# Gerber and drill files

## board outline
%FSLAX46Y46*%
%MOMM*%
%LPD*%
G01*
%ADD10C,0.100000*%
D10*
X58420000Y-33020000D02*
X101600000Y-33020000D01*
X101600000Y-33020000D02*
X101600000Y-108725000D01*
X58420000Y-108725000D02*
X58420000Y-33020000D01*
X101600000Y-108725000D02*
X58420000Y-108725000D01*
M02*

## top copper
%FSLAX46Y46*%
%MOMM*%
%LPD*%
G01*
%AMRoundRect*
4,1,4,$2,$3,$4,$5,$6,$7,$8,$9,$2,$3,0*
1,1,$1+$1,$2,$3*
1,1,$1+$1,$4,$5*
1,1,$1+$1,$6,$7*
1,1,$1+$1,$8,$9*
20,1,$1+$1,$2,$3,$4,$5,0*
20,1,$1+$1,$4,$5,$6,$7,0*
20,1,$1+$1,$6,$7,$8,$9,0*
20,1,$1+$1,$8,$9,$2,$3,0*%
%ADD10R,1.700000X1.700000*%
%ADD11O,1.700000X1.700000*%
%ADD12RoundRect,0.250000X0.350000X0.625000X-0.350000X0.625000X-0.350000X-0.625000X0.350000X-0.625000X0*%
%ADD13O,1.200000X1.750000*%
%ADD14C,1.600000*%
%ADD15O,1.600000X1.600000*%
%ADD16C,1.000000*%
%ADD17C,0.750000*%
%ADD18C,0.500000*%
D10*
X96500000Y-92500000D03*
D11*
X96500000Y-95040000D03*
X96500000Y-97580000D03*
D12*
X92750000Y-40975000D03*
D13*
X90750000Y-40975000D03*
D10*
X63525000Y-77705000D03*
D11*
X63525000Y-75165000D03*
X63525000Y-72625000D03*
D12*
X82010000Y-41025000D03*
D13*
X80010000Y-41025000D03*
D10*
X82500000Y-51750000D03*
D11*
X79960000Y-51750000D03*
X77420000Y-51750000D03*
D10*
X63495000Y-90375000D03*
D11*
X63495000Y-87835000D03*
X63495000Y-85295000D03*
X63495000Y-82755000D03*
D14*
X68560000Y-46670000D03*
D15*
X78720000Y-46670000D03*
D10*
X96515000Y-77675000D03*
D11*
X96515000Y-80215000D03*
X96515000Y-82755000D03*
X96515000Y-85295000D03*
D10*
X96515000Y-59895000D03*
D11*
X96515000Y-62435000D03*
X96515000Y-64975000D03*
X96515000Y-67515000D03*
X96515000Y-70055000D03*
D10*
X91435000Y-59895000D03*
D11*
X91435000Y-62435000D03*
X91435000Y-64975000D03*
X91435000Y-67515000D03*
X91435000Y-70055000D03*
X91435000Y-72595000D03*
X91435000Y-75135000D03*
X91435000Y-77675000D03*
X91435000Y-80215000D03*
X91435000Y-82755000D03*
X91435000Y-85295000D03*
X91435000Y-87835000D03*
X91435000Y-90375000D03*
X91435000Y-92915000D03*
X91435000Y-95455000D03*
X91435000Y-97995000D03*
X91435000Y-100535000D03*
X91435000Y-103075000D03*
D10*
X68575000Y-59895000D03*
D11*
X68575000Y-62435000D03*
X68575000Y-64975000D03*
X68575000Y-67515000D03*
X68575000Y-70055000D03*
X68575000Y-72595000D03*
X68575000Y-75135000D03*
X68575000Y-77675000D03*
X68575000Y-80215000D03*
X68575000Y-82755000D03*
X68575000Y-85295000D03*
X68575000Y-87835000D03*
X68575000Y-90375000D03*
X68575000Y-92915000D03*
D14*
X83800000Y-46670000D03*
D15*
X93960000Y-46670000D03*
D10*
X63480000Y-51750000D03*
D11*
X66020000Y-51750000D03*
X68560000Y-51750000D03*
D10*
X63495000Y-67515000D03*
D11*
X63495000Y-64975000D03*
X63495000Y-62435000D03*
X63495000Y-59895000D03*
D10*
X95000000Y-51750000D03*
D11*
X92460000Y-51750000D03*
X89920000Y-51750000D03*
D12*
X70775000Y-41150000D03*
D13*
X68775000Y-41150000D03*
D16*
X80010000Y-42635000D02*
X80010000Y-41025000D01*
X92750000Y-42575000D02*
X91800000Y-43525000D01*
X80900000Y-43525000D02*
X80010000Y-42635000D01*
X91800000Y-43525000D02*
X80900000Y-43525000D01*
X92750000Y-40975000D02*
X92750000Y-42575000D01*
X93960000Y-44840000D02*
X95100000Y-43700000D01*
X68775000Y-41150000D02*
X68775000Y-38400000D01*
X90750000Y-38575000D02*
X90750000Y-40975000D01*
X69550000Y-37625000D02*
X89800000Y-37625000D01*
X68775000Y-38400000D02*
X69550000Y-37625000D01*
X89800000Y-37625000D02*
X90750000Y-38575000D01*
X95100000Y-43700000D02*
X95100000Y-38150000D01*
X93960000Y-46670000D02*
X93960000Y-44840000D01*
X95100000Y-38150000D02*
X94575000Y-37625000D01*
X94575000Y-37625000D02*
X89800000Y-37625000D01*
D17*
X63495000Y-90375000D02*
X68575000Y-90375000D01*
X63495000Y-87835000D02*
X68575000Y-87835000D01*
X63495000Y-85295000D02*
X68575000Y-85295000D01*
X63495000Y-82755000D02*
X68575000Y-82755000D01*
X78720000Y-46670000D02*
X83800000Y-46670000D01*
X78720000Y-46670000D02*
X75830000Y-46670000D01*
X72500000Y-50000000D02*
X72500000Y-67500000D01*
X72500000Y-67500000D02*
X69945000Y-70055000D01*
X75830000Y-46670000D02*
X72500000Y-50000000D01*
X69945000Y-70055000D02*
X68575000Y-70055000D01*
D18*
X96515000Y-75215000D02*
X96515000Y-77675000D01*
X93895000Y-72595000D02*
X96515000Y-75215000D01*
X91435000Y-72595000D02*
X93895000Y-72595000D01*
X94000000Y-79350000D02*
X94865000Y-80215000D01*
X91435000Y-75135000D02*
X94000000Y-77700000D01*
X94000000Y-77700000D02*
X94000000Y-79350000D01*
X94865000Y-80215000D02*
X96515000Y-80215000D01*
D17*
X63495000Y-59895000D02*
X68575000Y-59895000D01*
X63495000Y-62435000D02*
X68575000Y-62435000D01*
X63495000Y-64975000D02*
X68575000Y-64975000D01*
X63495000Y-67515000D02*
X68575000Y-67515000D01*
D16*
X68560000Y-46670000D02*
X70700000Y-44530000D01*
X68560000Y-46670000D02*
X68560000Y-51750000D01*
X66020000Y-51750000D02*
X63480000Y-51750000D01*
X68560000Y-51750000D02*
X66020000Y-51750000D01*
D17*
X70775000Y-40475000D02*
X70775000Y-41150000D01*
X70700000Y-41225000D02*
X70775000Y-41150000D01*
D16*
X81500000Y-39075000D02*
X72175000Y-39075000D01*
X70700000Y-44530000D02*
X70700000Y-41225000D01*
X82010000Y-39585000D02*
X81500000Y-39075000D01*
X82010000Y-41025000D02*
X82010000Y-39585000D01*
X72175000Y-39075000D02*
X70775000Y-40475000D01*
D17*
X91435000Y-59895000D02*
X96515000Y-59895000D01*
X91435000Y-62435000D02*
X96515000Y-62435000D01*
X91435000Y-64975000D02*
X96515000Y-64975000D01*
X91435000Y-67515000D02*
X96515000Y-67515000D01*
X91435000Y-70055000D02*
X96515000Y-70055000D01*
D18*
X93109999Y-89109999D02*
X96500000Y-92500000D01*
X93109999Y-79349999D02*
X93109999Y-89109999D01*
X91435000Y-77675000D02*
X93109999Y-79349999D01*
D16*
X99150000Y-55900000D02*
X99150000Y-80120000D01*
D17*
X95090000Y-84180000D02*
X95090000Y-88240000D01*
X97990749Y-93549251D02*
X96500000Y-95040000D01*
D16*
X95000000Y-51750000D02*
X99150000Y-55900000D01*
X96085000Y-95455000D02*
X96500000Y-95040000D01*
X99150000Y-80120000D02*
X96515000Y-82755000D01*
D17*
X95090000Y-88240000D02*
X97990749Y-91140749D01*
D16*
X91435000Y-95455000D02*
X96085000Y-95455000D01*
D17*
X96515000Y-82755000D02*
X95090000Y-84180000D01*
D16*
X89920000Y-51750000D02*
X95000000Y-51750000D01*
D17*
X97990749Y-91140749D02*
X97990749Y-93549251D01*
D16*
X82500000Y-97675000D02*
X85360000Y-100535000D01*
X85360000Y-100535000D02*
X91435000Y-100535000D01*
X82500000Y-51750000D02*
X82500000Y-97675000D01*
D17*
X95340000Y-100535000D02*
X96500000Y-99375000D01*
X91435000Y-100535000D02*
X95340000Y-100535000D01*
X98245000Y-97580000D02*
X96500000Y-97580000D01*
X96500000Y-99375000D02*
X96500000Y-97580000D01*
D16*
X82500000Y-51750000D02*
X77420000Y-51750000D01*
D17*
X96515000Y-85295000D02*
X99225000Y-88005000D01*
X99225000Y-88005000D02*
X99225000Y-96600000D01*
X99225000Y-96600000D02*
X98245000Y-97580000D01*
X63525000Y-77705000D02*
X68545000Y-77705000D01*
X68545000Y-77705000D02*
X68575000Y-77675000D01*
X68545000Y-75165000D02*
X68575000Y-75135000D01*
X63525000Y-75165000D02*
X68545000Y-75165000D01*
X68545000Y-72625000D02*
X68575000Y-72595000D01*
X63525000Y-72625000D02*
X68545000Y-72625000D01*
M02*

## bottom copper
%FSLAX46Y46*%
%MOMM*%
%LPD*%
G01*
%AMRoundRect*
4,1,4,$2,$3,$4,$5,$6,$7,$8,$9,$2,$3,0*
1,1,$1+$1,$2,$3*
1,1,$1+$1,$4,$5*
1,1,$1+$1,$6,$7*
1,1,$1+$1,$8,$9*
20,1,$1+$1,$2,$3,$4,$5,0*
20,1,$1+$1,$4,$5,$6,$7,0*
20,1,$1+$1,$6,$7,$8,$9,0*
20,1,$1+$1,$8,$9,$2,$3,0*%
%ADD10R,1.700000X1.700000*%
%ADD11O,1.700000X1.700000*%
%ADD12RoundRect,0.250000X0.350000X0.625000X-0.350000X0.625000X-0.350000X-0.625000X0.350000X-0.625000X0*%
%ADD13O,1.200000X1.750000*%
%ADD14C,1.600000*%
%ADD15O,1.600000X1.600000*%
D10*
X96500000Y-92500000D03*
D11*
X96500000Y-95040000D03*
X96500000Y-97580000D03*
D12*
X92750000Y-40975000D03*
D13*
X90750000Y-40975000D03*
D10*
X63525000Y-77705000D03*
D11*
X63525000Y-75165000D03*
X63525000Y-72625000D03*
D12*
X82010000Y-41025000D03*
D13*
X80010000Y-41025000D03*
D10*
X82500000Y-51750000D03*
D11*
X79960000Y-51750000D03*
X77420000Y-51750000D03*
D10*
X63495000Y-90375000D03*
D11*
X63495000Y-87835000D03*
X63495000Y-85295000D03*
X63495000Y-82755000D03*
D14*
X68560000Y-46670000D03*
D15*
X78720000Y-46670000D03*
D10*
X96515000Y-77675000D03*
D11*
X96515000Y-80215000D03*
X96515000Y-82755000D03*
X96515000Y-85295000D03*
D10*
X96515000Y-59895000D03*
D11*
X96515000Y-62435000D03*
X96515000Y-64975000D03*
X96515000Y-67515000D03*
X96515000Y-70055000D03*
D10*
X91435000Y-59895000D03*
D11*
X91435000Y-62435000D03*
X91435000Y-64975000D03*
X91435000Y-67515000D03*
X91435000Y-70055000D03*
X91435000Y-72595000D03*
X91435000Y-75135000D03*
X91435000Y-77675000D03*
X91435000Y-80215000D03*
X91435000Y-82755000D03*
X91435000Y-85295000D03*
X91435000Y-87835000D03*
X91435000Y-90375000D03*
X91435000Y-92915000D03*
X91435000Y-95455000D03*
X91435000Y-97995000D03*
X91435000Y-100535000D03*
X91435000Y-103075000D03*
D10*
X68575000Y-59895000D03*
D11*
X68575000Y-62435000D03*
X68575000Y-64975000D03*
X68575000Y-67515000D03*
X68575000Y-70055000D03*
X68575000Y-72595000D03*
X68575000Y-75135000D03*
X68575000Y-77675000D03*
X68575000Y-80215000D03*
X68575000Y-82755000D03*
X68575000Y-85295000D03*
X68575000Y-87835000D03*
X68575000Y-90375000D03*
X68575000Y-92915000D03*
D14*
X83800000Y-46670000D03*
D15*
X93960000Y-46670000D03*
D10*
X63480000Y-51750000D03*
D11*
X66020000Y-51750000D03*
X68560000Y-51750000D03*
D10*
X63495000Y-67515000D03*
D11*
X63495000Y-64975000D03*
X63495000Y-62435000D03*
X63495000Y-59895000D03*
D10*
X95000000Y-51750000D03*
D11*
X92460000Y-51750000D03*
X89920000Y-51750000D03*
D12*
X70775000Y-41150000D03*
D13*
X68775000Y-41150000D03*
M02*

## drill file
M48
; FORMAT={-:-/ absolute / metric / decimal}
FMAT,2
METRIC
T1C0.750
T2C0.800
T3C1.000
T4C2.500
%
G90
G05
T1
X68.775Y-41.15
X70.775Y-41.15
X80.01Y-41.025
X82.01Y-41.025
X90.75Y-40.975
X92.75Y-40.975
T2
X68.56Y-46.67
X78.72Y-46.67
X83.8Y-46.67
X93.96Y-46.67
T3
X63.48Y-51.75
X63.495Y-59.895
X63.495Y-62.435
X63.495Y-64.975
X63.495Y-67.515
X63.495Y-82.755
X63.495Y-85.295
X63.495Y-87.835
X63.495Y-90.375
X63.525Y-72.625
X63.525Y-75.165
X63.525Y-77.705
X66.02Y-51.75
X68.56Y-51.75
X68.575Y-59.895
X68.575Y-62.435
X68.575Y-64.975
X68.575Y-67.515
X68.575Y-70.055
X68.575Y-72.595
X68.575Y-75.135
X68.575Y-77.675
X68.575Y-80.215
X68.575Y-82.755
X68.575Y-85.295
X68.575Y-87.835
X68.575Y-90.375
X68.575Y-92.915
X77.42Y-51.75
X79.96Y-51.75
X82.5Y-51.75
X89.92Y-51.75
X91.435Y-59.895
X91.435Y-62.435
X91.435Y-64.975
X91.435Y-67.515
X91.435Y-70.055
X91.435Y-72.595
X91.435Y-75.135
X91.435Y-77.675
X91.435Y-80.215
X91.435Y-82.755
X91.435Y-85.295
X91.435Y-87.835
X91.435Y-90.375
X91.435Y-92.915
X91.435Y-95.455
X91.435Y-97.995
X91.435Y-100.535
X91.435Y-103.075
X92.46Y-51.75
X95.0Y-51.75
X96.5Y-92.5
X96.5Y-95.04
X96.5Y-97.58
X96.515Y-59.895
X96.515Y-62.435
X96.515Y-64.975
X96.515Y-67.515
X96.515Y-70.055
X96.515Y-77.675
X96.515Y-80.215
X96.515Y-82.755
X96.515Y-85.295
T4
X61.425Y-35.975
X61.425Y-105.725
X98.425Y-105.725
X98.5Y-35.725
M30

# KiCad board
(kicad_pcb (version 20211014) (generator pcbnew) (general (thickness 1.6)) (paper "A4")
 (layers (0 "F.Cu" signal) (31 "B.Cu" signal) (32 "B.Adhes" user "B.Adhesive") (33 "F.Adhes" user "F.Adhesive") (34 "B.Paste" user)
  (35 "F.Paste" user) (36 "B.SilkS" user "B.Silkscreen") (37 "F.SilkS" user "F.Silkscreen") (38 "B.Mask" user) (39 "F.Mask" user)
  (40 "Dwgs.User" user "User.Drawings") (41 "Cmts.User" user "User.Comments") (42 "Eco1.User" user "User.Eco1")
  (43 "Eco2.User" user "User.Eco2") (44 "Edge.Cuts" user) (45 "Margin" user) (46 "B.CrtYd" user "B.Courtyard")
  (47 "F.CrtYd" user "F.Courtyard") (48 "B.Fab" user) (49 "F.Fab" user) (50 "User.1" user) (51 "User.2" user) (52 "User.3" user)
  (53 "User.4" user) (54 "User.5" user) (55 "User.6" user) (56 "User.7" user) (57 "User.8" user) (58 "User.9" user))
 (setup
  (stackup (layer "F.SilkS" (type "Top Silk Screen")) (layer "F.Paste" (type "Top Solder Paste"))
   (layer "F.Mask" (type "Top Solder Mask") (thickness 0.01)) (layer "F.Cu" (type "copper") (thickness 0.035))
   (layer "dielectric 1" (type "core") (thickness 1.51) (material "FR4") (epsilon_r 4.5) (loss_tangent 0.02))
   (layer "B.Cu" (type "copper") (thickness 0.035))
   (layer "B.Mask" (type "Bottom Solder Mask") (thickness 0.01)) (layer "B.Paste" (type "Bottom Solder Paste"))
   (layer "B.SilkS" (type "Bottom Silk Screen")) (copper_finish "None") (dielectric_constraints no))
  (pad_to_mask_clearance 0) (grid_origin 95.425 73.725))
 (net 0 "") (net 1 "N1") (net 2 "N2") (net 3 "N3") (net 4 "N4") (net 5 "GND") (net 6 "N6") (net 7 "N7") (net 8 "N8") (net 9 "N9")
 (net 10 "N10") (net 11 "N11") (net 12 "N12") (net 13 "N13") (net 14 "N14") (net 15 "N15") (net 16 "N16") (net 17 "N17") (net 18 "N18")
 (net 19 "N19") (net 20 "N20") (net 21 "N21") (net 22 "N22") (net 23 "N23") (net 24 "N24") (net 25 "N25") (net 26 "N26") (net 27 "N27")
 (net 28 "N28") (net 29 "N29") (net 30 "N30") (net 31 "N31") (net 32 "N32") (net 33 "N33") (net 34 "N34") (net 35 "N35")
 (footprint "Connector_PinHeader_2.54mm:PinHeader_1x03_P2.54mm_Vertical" (layer "F.Cu") (at 96.5 92.5)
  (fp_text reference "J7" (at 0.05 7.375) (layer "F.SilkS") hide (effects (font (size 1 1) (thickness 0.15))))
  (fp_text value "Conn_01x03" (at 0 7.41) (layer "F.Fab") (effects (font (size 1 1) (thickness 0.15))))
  (pad "1" thru_hole rect (at 0 0) (size 1.7 1.7) (drill 1) (layers *.Cu *.Mask) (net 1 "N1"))
  (pad "2" thru_hole oval (at 0 2.54) (size 1.7 1.7) (drill 1) (layers *.Cu *.Mask) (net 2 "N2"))
  (pad "3" thru_hole oval (at 0 5.08) (size 1.7 1.7) (drill 1) (layers *.Cu *.Mask) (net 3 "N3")))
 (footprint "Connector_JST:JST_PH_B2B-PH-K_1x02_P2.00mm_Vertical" (layer "F.Cu") (at 92.75 40.975 180)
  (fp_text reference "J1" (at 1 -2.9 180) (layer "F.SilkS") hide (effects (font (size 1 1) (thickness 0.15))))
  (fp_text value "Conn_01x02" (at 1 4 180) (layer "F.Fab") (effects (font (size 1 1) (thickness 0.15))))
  (pad "1" thru_hole roundrect (at 0 0 180) (size 1.2 1.75) (drill 0.75) (layers *.Cu *.Mask) (roundrect_rratio 0.208333) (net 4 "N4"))
  (pad "2" thru_hole oval (at 2 0 180) (size 1.2 1.75) (drill 0.75) (layers *.Cu *.Mask) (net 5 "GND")))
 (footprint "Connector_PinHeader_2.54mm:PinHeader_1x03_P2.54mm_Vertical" (layer "F.Cu") (at 63.525 77.705 180)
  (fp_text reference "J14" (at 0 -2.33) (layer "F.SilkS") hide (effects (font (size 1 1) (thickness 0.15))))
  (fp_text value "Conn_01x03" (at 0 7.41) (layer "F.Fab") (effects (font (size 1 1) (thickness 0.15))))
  (pad "1" thru_hole rect (at 0 0 180) (size 1.7 1.7) (drill 1) (layers *.Cu *.Mask) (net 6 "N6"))
  (pad "2" thru_hole oval (at 0 2.54 180) (size 1.7 1.7) (drill 1) (layers *.Cu *.Mask) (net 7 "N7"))
  (pad "3" thru_hole oval (at 0 5.08 180) (size 1.7 1.7) (drill 1) (layers *.Cu *.Mask) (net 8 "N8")))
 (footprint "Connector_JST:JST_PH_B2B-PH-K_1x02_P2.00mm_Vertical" (layer "F.Cu") (at 82.01 41.025 180)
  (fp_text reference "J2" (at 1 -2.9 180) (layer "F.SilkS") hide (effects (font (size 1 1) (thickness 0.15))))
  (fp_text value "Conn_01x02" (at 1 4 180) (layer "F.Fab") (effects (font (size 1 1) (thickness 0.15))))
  (pad "1" thru_hole roundrect (at 0 0 180) (size 1.2 1.75) (drill 0.75) (layers *.Cu *.Mask) (roundrect_rratio 0.208333) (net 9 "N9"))
  (pad "2" thru_hole oval (at 2 0 180) (size 1.2 1.75) (drill 0.75) (layers *.Cu *.Mask) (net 4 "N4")))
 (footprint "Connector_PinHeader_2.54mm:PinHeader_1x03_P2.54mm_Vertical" (layer "F.Cu") (at 82.5 51.75 -90)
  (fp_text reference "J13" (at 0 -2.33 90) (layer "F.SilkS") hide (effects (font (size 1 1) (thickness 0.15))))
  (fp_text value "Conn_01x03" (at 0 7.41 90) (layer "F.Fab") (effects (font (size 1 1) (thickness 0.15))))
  (pad "1" thru_hole rect (at 0 0 270) (size 1.7 1.7) (drill 1) (layers *.Cu *.Mask) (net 3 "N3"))
  (pad "2" thru_hole oval (at 0 2.54 270) (size 1.7 1.7) (drill 1) (layers *.Cu *.Mask) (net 3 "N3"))
  (pad "3" thru_hole oval (at 0 5.08 270) (size 1.7 1.7) (drill 1) (layers *.Cu *.Mask) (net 3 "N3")))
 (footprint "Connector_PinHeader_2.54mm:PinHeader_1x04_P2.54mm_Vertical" (layer "F.Cu") (at 63.495 90.375 180)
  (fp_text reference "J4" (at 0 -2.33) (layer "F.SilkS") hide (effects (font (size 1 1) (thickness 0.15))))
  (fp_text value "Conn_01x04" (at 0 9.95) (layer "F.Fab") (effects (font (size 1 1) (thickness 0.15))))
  (pad "1" thru_hole rect (at 0 0 180) (size 1.7 1.7) (drill 1) (layers *.Cu *.Mask) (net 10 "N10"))
  (pad "2" thru_hole oval (at 0 2.54 180) (size 1.7 1.7) (drill 1) (layers *.Cu *.Mask) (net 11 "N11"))
  (pad "3" thru_hole oval (at 0 5.08 180) (size 1.7 1.7) (drill 1) (layers *.Cu *.Mask) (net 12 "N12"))
  (pad "4" thru_hole oval (at 0 7.62 180) (size 1.7 1.7) (drill 1) (layers *.Cu *.Mask) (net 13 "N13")))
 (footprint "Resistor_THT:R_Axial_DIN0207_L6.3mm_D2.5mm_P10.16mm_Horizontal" (layer "F.Cu") (at 68.56 46.67)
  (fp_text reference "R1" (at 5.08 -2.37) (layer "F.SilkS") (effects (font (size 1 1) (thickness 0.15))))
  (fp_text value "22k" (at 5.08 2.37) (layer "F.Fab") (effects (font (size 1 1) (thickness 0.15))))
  (pad "1" thru_hole circle (at 0 0) (size 1.6 1.6) (drill 0.8) (layers *.Cu *.Mask) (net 9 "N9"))
  (pad "2" thru_hole oval (at 10.16 0) (size 1.6 1.6) (drill 0.8) (layers *.Cu *.Mask) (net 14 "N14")))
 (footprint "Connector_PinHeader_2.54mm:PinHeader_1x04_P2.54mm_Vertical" (layer "F.Cu") (at 96.515 77.675)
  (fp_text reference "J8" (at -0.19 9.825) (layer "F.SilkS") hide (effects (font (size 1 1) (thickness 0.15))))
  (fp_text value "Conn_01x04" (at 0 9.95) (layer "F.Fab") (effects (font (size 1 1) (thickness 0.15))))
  (pad "1" thru_hole rect (at 0 0) (size 1.7 1.7) (drill 1) (layers *.Cu *.Mask) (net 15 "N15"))
  (pad "2" thru_hole oval (at 0 2.54) (size 1.7 1.7) (drill 1) (layers *.Cu *.Mask) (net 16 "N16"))
  (pad "3" thru_hole oval (at 0 5.08) (size 1.7 1.7) (drill 1) (layers *.Cu *.Mask) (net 2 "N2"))
  (pad "4" thru_hole oval (at 0 7.62) (size 1.7 1.7) (drill 1) (layers *.Cu *.Mask) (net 3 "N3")))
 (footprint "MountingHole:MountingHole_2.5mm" (layer "F.Cu") (at 98.425 35.725)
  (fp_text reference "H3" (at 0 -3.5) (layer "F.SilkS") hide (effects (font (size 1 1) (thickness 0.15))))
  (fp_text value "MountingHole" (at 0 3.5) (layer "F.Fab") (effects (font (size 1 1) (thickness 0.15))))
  (pad "" np_thru_hole circle (at 0.075 0) (size 2.5 2.5) (drill 2.5) (layers F&B.Cu *.Mask)))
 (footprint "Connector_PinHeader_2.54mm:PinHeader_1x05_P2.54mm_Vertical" (layer "F.Cu") (at 96.515 59.895)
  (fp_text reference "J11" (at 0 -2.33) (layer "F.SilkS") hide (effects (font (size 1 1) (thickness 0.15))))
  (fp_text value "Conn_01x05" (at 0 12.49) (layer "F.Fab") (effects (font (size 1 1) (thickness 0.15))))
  (pad "1" thru_hole rect (at 0 0) (size 1.7 1.7) (drill 1) (layers *.Cu *.Mask) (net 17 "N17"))
  (pad "2" thru_hole oval (at 0 2.54) (size 1.7 1.7) (drill 1) (layers *.Cu *.Mask) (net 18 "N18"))
  (pad "3" thru_hole oval (at 0 5.08) (size 1.7 1.7) (drill 1) (layers *.Cu *.Mask) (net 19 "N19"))
  (pad "4" thru_hole oval (at 0 7.62) (size 1.7 1.7) (drill 1) (layers *.Cu *.Mask) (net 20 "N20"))
  (pad "5" thru_hole oval (at 0 10.16) (size 1.7 1.7) (drill 1) (layers *.Cu *.Mask) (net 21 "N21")))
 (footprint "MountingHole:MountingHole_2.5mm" (layer "F.Cu") (at 61.425 35.975)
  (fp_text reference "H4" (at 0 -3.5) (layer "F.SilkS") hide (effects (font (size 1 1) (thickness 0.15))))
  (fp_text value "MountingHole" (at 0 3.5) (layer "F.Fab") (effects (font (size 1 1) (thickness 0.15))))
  (pad "" np_thru_hole circle (at 0 0) (size 2.5 2.5) (drill 2.5) (layers *.Cu *.Mask)))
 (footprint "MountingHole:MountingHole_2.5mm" (layer "F.Cu") (at 98.425 105.725)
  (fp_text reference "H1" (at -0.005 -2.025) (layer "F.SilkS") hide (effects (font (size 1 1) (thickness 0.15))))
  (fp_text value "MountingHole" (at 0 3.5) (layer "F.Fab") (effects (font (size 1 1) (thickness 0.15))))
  (pad "" np_thru_hole circle (at 0 0) (size 2.5 2.5) (drill 2.5) (layers *.Cu *.Mask)))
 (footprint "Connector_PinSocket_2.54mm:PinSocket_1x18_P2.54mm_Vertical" (layer "F.Cu") (at 91.435 59.895)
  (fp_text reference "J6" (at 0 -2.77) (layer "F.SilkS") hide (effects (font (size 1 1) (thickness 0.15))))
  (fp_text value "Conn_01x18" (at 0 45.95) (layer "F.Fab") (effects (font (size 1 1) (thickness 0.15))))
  (pad "1" thru_hole rect (at 0 0) (size 1.7 1.7) (drill 1) (layers *.Cu *.Mask) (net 17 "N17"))
  (pad "2" thru_hole oval (at 0 2.54) (size 1.7 1.7) (drill 1) (layers *.Cu *.Mask) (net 18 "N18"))
  (pad "3" thru_hole oval (at 0 5.08) (size 1.7 1.7) (drill 1) (layers *.Cu *.Mask) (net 19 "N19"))
  (pad "4" thru_hole oval (at 0 7.62) (size 1.7 1.7) (drill 1) (layers *.Cu *.Mask) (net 20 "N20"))
  (pad "5" thru_hole oval (at 0 10.16) (size 1.7 1.7) (drill 1) (layers *.Cu *.Mask) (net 21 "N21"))
  (pad "6" thru_hole oval (at 0 12.7) (size 1.7 1.7) (drill 1) (layers *.Cu *.Mask) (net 15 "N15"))
  (pad "7" thru_hole oval (at 0 15.24) (size 1.7 1.7) (drill 1) (layers *.Cu *.Mask) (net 16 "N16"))
  (pad "8" thru_hole oval (at 0 17.78) (size 1.7 1.7) (drill 1) (layers *.Cu *.Mask) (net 1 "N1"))
  (pad "9" thru_hole oval (at 0 20.32) (size 1.7 1.7) (drill 1) (layers *.Cu *.Mask) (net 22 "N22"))
  (pad "10" thru_hole oval (at 0 22.86) (size 1.7 1.7) (drill 1) (layers *.Cu *.Mask) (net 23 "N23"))
  (pad "11" thru_hole oval (at 0 25.4) (size 1.7 1.7) (drill 1) (layers *.Cu *.Mask) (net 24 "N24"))
  (pad "12" thru_hole oval (at 0 27.94) (size 1.7 1.7) (drill 1) (layers *.Cu *.Mask) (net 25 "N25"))
  (pad "13" thru_hole oval (at 0 30.48) (size 1.7 1.7) (drill 1) (layers *.Cu *.Mask) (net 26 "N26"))
  (pad "14" thru_hole oval (at 0 33.02) (size 1.7 1.7) (drill 1) (layers *.Cu *.Mask) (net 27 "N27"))
  (pad "15" thru_hole oval (at 0 35.56) (size 1.7 1.7) (drill 1) (layers *.Cu *.Mask) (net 2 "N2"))
  (pad "16" thru_hole oval (at 0 38.1) (size 1.7 1.7) (drill 1) (layers *.Cu *.Mask) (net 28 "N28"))
  (pad "17" thru_hole oval (at 0 40.64) (size 1.7 1.7) (drill 1) (layers *.Cu *.Mask) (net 3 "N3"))
  (pad "18" thru_hole oval (at 0 43.18) (size 1.7 1.7) (drill 1) (layers *.Cu *.Mask) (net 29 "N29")))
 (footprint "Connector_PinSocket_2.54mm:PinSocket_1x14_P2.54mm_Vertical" (layer "F.Cu") (at 68.575 59.895)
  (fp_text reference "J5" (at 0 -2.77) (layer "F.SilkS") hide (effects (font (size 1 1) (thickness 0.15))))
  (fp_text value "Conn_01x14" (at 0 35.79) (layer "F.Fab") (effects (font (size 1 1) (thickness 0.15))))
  (pad "1" thru_hole rect (at 0 0) (size 1.7 1.7) (drill 1) (layers *.Cu *.Mask) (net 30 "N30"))
  (pad "2" thru_hole oval (at 0 2.54) (size 1.7 1.7) (drill 1) (layers *.Cu *.Mask) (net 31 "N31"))
  (pad "3" thru_hole oval (at 0 5.08) (size 1.7 1.7) (drill 1) (layers *.Cu *.Mask) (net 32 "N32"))
  (pad "4" thru_hole oval (at 0 7.62) (size 1.7 1.7) (drill 1) (layers *.Cu *.Mask) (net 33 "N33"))
  (pad "5" thru_hole oval (at 0 10.16) (size 1.7 1.7) (drill 1) (layers *.Cu *.Mask) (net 14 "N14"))
  (pad "6" thru_hole oval (at 0 12.7) (size 1.7 1.7) (drill 1) (layers *.Cu *.Mask) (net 8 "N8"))
  (pad "7" thru_hole oval (at 0 15.24) (size 1.7 1.7) (drill 1) (layers *.Cu *.Mask) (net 7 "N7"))
  (pad "8" thru_hole oval (at 0 17.78) (size 1.7 1.7) (drill 1) (layers *.Cu *.Mask) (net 6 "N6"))
  (pad "9" thru_hole oval (at 0 20.32) (size 1.7 1.7) (drill 1) (layers *.Cu *.Mask) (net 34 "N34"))
  (pad "10" thru_hole oval (at 0 22.86) (size 1.7 1.7) (drill 1) (layers *.Cu *.Mask) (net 13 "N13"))
  (pad "11" thru_hole oval (at 0 25.4) (size 1.7 1.7) (drill 1) (layers *.Cu *.Mask) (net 12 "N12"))
  (pad "12" thru_hole oval (at 0 27.94) (size 1.7 1.7) (drill 1) (layers *.Cu *.Mask) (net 11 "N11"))
  (pad "13" thru_hole oval (at 0 30.48) (size 1.7 1.7) (drill 1) (layers *.Cu *.Mask) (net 10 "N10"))
  (pad "14" thru_hole oval (at 0 33.02) (size 1.7 1.7) (drill 1) (layers *.Cu *.Mask) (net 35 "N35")))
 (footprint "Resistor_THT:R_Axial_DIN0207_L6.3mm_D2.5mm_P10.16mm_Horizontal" (layer "F.Cu") (at 83.8 46.67)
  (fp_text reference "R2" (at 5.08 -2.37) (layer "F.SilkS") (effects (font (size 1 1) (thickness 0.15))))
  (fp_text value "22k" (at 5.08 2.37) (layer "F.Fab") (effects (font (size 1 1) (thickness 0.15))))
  (pad "1" thru_hole circle (at 0 0) (size 1.6 1.6) (drill 0.8) (layers *.Cu *.Mask) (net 14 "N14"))
  (pad "2" thru_hole oval (at 10.16 0) (size 1.6 1.6) (drill 0.8) (layers *.Cu *.Mask) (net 5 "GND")))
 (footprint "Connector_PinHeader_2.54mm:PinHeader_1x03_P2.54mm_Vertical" (layer "F.Cu") (at 63.48 51.75 90)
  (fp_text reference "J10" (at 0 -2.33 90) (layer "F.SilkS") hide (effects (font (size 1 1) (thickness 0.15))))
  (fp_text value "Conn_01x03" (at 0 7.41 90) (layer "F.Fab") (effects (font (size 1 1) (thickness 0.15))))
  (pad "1" thru_hole rect (at 0 0 90) (size 1.7 1.7) (drill 1) (layers *.Cu *.Mask) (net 9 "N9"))
  (pad "2" thru_hole oval (at 0 2.54 90) (size 1.7 1.7) (drill 1) (layers *.Cu *.Mask) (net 9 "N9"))
  (pad "3" thru_hole oval (at 0 5.08 90) (size 1.7 1.7) (drill 1) (layers *.Cu *.Mask) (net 9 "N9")))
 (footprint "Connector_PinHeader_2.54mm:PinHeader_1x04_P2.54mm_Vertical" (layer "F.Cu") (at 63.495 67.515 180)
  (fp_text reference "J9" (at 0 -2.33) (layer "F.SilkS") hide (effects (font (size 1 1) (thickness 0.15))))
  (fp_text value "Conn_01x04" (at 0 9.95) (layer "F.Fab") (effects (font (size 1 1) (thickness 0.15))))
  (pad "1" thru_hole rect (at 0 0 180) (size 1.7 1.7) (drill 1) (layers *.Cu *.Mask) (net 33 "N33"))
  (pad "2" thru_hole oval (at 0 2.54 180) (size 1.7 1.7) (drill 1) (layers *.Cu *.Mask) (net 32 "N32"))
  (pad "3" thru_hole oval (at 0 5.08 180) (size 1.7 1.7) (drill 1) (layers *.Cu *.Mask) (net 31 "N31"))
  (pad "4" thru_hole oval (at 0 7.62 180) (size 1.7 1.7) (drill 1) (layers *.Cu *.Mask) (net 30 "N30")))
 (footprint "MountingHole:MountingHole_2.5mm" (layer "F.Cu") (at 61.425 105.725)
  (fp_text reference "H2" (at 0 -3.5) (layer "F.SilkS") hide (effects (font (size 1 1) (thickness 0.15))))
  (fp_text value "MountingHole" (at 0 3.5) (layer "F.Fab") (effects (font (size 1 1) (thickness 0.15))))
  (pad "" np_thru_hole circle (at 0 0) (size 2.5 2.5) (drill 2.5) (layers *.Cu *.Mask)))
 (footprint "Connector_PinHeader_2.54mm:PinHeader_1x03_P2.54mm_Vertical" (layer "F.Cu") (at 95 51.75 -90)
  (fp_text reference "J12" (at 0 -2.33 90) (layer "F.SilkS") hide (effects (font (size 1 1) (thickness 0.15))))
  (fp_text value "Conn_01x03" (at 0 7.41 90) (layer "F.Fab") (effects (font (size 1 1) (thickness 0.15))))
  (pad "1" thru_hole rect (at 0 0 270) (size 1.7 1.7) (drill 1) (layers *.Cu *.Mask) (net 2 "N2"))
  (pad "2" thru_hole oval (at 0 2.54 270) (size 1.7 1.7) (drill 1) (layers *.Cu *.Mask) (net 2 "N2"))
  (pad "3" thru_hole oval (at 0 5.08 270) (size 1.7 1.7) (drill 1) (layers *.Cu *.Mask) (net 2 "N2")))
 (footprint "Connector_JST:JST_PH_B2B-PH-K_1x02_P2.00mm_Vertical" (layer "F.Cu") (at 70.775 41.15 180)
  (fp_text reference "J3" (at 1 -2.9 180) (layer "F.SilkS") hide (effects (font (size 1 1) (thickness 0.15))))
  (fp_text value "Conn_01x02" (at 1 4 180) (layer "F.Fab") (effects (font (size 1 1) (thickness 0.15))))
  (pad "1" thru_hole roundrect (at 0 0 180) (size 1.2 1.75) (drill 0.75) (layers *.Cu *.Mask) (roundrect_rratio 0.208333) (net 9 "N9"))
  (pad "2" thru_hole oval (at 2 0 180) (size 1.2 1.75) (drill 0.75) (layers *.Cu *.Mask) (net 5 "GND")))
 (gr_line (start 58.42 33.02) (end 101.6 33.02) (layer "Edge.Cuts") (width 0.1))
 (gr_line (start 101.6 33.02) (end 101.6 108.725) (layer "Edge.Cuts") (width 0.1))
 (gr_line (start 58.42 108.725) (end 58.42 33.02) (layer "Edge.Cuts") (width 0.1))
 (gr_line (start 101.6 108.725) (end 58.42 108.725) (layer "Edge.Cuts") (width 0.1))
 (segment (start 80.01 42.635) (end 80.01 41.025) (width 1) (layer "F.Cu") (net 4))
 (segment (start 92.75 42.575) (end 91.8 43.525) (width 1) (layer "F.Cu") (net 4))
 (segment (start 80.9 43.525) (end 80.01 42.635) (width 1) (layer "F.Cu") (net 4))
 (segment (start 91.8 43.525) (end 80.9 43.525) (width 1) (layer "F.Cu") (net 4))
 (segment (start 92.75 40.975) (end 92.75 42.575) (width 1) (layer "F.Cu") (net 4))
 (segment (start 93.96 44.84) (end 95.1 43.7) (width 1) (layer "F.Cu") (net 5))
 (segment (start 68.775 41.15) (end 68.775 38.4) (width 1) (layer "F.Cu") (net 5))
 (segment (start 90.75 38.575) (end 90.75 40.975) (width 1) (layer "F.Cu") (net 5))
 (segment (start 69.55 37.625) (end 89.8 37.625) (width 1) (layer "F.Cu") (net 5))
 (segment (start 68.775 38.4) (end 69.55 37.625) (width 1) (layer "F.Cu") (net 5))
 (segment (start 89.8 37.625) (end 90.75 38.575) (width 1) (layer "F.Cu") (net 5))
 (segment (start 95.1 43.7) (end 95.1 38.15) (width 1) (layer "F.Cu") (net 5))
 (segment (start 93.96 46.67) (end 93.96 44.84) (width 1) (layer "F.Cu") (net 5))
 (segment (start 95.1 38.15) (end 94.575 37.625) (width 1) (layer "F.Cu") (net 5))
 (segment (start 94.575 37.625) (end 89.8 37.625) (width 1) (layer "F.Cu") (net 5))
 (segment (start 63.495 90.375) (end 68.575 90.375) (width 0.75) (layer "F.Cu") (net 10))
 (segment (start 63.495 87.835) (end 68.575 87.835) (width 0.75) (layer "F.Cu") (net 11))
 (segment (start 63.495 85.295) (end 68.575 85.295) (width 0.75) (layer "F.Cu") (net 12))
 (segment (start 63.495 82.755) (end 68.575 82.755) (width 0.75) (layer "F.Cu") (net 13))
 (segment (start 78.72 46.67) (end 83.8 46.67) (width 0.75) (layer "F.Cu") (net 14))
 (segment (start 78.72 46.67) (end 75.83 46.67) (width 0.75) (layer "F.Cu") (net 14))
 (segment (start 72.5 50) (end 72.5 67.5) (width 0.75) (layer "F.Cu") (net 14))
 (segment (start 72.5 67.5) (end 69.945 70.055) (width 0.75) (layer "F.Cu") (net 14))
 (segment (start 75.83 46.67) (end 72.5 50) (width 0.75) (layer "F.Cu") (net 14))
 (segment (start 69.945 70.055) (end 68.575 70.055) (width 0.75) (layer "F.Cu") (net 14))
 (segment (start 96.515 75.215) (end 96.515 77.675) (width 0.5) (layer "F.Cu") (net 15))
 (segment (start 93.895 72.595) (end 96.515 75.215) (width 0.5) (layer "F.Cu") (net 15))
 (segment (start 91.435 72.595) (end 93.895 72.595) (width 0.5) (layer "F.Cu") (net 15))
 (segment (start 94 79.35) (end 94.865 80.215) (width 0.5) (layer "F.Cu") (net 16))
 (segment (start 91.435 75.135) (end 94 77.7) (width 0.5) (layer "F.Cu") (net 16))
 (segment (start 94 77.7) (end 94 79.35) (width 0.5) (layer "F.Cu") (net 16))
 (segment (start 94.865 80.215) (end 96.515 80.215) (width 0.5) (layer "F.Cu") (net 16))
 (segment (start 63.495 59.895) (end 68.575 59.895) (width 0.75) (layer "F.Cu") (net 30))
 (segment (start 63.495 62.435) (end 68.575 62.435) (width 0.75) (layer "F.Cu") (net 31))
 (segment (start 63.495 64.975) (end 68.575 64.975) (width 0.75) (layer "F.Cu") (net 32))
 (segment (start 63.495 67.515) (end 68.575 67.515) (width 0.75) (layer "F.Cu") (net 33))
 (segment (start 68.56 46.67) (end 70.7 44.53) (width 1) (layer "F.Cu") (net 9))
 (segment (start 68.56 46.67) (end 68.56 51.75) (width 1) (layer "F.Cu") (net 9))
 (segment (start 66.02 51.75) (end 63.48 51.75) (width 1) (layer "F.Cu") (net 9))
 (segment (start 68.56 51.75) (end 66.02 51.75) (width 1) (layer "F.Cu") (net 9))
 (segment (start 70.775 40.475) (end 70.775 41.15) (width 0.75) (layer "F.Cu") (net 9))
 (segment (start 70.7 41.225) (end 70.775 41.15) (width 0.75) (layer "F.Cu") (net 9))
 (segment (start 81.5 39.075) (end 72.175 39.075) (width 1) (layer "F.Cu") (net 9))
 (segment (start 70.7 44.53) (end 70.7 41.225) (width 1) (layer "F.Cu") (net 9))
 (segment (start 82.01 39.585) (end 81.5 39.075) (width 1) (layer "F.Cu") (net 9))
 (segment (start 82.01 41.025) (end 82.01 39.585) (width 1) (layer "F.Cu") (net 9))
 (segment (start 72.175 39.075) (end 70.775 40.475) (width 1) (layer "F.Cu") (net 9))
 (segment (start 91.435 59.895) (end 96.515 59.895) (width 0.75) (layer "F.Cu") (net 17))
 (segment (start 91.435 62.435) (end 96.515 62.435) (width 0.75) (layer "F.Cu") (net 18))
 (segment (start 91.435 64.975) (end 96.515 64.975) (width 0.75) (layer "F.Cu") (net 19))
 (segment (start 91.435 67.515) (end 96.515 67.515) (width 0.75) (layer "F.Cu") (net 20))
 (segment (start 91.435 70.055) (end 96.515 70.055) (width 0.75) (layer "F.Cu") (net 21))
 (segment (start 93.109999 89.109999) (end 96.5 92.5) (width 0.5) (layer "F.Cu") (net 1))
 (segment (start 93.109999 79.349999) (end 93.109999 89.109999) (width 0.5) (layer "F.Cu") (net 1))
 (segment (start 91.435 77.675) (end 93.109999 79.349999) (width 0.5) (layer "F.Cu") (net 1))
 (segment (start 99.15 55.9) (end 99.15 80.12) (width 1) (layer "F.Cu") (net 2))
 (segment (start 95.09 84.18) (end 95.09 88.24) (width 0.75) (layer "F.Cu") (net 2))
 (segment (start 97.990749 93.549251) (end 96.5 95.04) (width 0.75) (layer "F.Cu") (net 2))
 (segment (start 95 51.75) (end 99.15 55.9) (width 1) (layer "F.Cu") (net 2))
 (segment (start 96.085 95.455) (end 96.5 95.04) (width 1) (layer "F.Cu") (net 2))
 (segment (start 99.15 80.12) (end 96.515 82.755) (width 1) (layer "F.Cu") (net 2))
 (segment (start 95.09 88.24) (end 97.990749 91.140749) (width 0.75) (layer "F.Cu") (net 2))
 (segment (start 91.435 95.455) (end 96.085 95.455) (width 1) (layer "F.Cu") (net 2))
 (segment (start 96.515 82.755) (end 95.09 84.18) (width 0.75) (layer "F.Cu") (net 2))
 (segment (start 89.92 51.75) (end 95 51.75) (width 1) (layer "F.Cu") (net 2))
 (segment (start 97.990749 91.140749) (end 97.990749 93.549251) (width 0.75) (layer "F.Cu") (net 2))
 (segment (start 82.5 97.675) (end 85.36 100.535) (width 1) (layer "F.Cu") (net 3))
 (segment (start 85.36 100.535) (end 91.435 100.535) (width 1) (layer "F.Cu") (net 3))
 (segment (start 82.5 51.75) (end 82.5 97.675) (width 1) (layer "F.Cu") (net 3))
 (segment (start 95.34 100.535) (end 96.5 99.375) (width 0.75) (layer "F.Cu") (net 3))
 (segment (start 91.435 100.535) (end 95.34 100.535) (width 0.75) (layer "F.Cu") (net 3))
 (segment (start 98.245 97.58) (end 96.5 97.58) (width 0.75) (layer "F.Cu") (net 3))
 (segment (start 96.5 99.375) (end 96.5 97.58) (width 0.75) (layer "F.Cu") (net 3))
 (segment (start 82.5 51.75) (end 77.42 51.75) (width 1) (layer "F.Cu") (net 3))
 (segment (start 96.515 85.295) (end 99.225 88.005) (width 0.75) (layer "F.Cu") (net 3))
 (segment (start 99.225 88.005) (end 99.225 96.6) (width 0.75) (layer "F.Cu") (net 3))
 (segment (start 99.225 96.6) (end 98.245 97.58) (width 0.75) (layer "F.Cu") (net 3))
 (segment (start 63.525 77.705) (end 68.545 77.705) (width 0.75) (layer "F.Cu") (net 6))
 (segment (start 68.545 77.705) (end 68.575 77.675) (width 0.75) (layer "F.Cu") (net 6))
 (segment (start 68.545 75.165) (end 68.575 75.135) (width 0.75) (layer "F.Cu") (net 7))
 (segment (start 63.525 75.165) (end 68.545 75.165) (width 0.75) (layer "F.Cu") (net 7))
 (segment (start 68.545 72.625) (end 68.575 72.595) (width 0.75) (layer "F.Cu") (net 8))
 (segment (start 63.525 72.625) (end 68.545 72.625) (width 0.75) (layer "F.Cu") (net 8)))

